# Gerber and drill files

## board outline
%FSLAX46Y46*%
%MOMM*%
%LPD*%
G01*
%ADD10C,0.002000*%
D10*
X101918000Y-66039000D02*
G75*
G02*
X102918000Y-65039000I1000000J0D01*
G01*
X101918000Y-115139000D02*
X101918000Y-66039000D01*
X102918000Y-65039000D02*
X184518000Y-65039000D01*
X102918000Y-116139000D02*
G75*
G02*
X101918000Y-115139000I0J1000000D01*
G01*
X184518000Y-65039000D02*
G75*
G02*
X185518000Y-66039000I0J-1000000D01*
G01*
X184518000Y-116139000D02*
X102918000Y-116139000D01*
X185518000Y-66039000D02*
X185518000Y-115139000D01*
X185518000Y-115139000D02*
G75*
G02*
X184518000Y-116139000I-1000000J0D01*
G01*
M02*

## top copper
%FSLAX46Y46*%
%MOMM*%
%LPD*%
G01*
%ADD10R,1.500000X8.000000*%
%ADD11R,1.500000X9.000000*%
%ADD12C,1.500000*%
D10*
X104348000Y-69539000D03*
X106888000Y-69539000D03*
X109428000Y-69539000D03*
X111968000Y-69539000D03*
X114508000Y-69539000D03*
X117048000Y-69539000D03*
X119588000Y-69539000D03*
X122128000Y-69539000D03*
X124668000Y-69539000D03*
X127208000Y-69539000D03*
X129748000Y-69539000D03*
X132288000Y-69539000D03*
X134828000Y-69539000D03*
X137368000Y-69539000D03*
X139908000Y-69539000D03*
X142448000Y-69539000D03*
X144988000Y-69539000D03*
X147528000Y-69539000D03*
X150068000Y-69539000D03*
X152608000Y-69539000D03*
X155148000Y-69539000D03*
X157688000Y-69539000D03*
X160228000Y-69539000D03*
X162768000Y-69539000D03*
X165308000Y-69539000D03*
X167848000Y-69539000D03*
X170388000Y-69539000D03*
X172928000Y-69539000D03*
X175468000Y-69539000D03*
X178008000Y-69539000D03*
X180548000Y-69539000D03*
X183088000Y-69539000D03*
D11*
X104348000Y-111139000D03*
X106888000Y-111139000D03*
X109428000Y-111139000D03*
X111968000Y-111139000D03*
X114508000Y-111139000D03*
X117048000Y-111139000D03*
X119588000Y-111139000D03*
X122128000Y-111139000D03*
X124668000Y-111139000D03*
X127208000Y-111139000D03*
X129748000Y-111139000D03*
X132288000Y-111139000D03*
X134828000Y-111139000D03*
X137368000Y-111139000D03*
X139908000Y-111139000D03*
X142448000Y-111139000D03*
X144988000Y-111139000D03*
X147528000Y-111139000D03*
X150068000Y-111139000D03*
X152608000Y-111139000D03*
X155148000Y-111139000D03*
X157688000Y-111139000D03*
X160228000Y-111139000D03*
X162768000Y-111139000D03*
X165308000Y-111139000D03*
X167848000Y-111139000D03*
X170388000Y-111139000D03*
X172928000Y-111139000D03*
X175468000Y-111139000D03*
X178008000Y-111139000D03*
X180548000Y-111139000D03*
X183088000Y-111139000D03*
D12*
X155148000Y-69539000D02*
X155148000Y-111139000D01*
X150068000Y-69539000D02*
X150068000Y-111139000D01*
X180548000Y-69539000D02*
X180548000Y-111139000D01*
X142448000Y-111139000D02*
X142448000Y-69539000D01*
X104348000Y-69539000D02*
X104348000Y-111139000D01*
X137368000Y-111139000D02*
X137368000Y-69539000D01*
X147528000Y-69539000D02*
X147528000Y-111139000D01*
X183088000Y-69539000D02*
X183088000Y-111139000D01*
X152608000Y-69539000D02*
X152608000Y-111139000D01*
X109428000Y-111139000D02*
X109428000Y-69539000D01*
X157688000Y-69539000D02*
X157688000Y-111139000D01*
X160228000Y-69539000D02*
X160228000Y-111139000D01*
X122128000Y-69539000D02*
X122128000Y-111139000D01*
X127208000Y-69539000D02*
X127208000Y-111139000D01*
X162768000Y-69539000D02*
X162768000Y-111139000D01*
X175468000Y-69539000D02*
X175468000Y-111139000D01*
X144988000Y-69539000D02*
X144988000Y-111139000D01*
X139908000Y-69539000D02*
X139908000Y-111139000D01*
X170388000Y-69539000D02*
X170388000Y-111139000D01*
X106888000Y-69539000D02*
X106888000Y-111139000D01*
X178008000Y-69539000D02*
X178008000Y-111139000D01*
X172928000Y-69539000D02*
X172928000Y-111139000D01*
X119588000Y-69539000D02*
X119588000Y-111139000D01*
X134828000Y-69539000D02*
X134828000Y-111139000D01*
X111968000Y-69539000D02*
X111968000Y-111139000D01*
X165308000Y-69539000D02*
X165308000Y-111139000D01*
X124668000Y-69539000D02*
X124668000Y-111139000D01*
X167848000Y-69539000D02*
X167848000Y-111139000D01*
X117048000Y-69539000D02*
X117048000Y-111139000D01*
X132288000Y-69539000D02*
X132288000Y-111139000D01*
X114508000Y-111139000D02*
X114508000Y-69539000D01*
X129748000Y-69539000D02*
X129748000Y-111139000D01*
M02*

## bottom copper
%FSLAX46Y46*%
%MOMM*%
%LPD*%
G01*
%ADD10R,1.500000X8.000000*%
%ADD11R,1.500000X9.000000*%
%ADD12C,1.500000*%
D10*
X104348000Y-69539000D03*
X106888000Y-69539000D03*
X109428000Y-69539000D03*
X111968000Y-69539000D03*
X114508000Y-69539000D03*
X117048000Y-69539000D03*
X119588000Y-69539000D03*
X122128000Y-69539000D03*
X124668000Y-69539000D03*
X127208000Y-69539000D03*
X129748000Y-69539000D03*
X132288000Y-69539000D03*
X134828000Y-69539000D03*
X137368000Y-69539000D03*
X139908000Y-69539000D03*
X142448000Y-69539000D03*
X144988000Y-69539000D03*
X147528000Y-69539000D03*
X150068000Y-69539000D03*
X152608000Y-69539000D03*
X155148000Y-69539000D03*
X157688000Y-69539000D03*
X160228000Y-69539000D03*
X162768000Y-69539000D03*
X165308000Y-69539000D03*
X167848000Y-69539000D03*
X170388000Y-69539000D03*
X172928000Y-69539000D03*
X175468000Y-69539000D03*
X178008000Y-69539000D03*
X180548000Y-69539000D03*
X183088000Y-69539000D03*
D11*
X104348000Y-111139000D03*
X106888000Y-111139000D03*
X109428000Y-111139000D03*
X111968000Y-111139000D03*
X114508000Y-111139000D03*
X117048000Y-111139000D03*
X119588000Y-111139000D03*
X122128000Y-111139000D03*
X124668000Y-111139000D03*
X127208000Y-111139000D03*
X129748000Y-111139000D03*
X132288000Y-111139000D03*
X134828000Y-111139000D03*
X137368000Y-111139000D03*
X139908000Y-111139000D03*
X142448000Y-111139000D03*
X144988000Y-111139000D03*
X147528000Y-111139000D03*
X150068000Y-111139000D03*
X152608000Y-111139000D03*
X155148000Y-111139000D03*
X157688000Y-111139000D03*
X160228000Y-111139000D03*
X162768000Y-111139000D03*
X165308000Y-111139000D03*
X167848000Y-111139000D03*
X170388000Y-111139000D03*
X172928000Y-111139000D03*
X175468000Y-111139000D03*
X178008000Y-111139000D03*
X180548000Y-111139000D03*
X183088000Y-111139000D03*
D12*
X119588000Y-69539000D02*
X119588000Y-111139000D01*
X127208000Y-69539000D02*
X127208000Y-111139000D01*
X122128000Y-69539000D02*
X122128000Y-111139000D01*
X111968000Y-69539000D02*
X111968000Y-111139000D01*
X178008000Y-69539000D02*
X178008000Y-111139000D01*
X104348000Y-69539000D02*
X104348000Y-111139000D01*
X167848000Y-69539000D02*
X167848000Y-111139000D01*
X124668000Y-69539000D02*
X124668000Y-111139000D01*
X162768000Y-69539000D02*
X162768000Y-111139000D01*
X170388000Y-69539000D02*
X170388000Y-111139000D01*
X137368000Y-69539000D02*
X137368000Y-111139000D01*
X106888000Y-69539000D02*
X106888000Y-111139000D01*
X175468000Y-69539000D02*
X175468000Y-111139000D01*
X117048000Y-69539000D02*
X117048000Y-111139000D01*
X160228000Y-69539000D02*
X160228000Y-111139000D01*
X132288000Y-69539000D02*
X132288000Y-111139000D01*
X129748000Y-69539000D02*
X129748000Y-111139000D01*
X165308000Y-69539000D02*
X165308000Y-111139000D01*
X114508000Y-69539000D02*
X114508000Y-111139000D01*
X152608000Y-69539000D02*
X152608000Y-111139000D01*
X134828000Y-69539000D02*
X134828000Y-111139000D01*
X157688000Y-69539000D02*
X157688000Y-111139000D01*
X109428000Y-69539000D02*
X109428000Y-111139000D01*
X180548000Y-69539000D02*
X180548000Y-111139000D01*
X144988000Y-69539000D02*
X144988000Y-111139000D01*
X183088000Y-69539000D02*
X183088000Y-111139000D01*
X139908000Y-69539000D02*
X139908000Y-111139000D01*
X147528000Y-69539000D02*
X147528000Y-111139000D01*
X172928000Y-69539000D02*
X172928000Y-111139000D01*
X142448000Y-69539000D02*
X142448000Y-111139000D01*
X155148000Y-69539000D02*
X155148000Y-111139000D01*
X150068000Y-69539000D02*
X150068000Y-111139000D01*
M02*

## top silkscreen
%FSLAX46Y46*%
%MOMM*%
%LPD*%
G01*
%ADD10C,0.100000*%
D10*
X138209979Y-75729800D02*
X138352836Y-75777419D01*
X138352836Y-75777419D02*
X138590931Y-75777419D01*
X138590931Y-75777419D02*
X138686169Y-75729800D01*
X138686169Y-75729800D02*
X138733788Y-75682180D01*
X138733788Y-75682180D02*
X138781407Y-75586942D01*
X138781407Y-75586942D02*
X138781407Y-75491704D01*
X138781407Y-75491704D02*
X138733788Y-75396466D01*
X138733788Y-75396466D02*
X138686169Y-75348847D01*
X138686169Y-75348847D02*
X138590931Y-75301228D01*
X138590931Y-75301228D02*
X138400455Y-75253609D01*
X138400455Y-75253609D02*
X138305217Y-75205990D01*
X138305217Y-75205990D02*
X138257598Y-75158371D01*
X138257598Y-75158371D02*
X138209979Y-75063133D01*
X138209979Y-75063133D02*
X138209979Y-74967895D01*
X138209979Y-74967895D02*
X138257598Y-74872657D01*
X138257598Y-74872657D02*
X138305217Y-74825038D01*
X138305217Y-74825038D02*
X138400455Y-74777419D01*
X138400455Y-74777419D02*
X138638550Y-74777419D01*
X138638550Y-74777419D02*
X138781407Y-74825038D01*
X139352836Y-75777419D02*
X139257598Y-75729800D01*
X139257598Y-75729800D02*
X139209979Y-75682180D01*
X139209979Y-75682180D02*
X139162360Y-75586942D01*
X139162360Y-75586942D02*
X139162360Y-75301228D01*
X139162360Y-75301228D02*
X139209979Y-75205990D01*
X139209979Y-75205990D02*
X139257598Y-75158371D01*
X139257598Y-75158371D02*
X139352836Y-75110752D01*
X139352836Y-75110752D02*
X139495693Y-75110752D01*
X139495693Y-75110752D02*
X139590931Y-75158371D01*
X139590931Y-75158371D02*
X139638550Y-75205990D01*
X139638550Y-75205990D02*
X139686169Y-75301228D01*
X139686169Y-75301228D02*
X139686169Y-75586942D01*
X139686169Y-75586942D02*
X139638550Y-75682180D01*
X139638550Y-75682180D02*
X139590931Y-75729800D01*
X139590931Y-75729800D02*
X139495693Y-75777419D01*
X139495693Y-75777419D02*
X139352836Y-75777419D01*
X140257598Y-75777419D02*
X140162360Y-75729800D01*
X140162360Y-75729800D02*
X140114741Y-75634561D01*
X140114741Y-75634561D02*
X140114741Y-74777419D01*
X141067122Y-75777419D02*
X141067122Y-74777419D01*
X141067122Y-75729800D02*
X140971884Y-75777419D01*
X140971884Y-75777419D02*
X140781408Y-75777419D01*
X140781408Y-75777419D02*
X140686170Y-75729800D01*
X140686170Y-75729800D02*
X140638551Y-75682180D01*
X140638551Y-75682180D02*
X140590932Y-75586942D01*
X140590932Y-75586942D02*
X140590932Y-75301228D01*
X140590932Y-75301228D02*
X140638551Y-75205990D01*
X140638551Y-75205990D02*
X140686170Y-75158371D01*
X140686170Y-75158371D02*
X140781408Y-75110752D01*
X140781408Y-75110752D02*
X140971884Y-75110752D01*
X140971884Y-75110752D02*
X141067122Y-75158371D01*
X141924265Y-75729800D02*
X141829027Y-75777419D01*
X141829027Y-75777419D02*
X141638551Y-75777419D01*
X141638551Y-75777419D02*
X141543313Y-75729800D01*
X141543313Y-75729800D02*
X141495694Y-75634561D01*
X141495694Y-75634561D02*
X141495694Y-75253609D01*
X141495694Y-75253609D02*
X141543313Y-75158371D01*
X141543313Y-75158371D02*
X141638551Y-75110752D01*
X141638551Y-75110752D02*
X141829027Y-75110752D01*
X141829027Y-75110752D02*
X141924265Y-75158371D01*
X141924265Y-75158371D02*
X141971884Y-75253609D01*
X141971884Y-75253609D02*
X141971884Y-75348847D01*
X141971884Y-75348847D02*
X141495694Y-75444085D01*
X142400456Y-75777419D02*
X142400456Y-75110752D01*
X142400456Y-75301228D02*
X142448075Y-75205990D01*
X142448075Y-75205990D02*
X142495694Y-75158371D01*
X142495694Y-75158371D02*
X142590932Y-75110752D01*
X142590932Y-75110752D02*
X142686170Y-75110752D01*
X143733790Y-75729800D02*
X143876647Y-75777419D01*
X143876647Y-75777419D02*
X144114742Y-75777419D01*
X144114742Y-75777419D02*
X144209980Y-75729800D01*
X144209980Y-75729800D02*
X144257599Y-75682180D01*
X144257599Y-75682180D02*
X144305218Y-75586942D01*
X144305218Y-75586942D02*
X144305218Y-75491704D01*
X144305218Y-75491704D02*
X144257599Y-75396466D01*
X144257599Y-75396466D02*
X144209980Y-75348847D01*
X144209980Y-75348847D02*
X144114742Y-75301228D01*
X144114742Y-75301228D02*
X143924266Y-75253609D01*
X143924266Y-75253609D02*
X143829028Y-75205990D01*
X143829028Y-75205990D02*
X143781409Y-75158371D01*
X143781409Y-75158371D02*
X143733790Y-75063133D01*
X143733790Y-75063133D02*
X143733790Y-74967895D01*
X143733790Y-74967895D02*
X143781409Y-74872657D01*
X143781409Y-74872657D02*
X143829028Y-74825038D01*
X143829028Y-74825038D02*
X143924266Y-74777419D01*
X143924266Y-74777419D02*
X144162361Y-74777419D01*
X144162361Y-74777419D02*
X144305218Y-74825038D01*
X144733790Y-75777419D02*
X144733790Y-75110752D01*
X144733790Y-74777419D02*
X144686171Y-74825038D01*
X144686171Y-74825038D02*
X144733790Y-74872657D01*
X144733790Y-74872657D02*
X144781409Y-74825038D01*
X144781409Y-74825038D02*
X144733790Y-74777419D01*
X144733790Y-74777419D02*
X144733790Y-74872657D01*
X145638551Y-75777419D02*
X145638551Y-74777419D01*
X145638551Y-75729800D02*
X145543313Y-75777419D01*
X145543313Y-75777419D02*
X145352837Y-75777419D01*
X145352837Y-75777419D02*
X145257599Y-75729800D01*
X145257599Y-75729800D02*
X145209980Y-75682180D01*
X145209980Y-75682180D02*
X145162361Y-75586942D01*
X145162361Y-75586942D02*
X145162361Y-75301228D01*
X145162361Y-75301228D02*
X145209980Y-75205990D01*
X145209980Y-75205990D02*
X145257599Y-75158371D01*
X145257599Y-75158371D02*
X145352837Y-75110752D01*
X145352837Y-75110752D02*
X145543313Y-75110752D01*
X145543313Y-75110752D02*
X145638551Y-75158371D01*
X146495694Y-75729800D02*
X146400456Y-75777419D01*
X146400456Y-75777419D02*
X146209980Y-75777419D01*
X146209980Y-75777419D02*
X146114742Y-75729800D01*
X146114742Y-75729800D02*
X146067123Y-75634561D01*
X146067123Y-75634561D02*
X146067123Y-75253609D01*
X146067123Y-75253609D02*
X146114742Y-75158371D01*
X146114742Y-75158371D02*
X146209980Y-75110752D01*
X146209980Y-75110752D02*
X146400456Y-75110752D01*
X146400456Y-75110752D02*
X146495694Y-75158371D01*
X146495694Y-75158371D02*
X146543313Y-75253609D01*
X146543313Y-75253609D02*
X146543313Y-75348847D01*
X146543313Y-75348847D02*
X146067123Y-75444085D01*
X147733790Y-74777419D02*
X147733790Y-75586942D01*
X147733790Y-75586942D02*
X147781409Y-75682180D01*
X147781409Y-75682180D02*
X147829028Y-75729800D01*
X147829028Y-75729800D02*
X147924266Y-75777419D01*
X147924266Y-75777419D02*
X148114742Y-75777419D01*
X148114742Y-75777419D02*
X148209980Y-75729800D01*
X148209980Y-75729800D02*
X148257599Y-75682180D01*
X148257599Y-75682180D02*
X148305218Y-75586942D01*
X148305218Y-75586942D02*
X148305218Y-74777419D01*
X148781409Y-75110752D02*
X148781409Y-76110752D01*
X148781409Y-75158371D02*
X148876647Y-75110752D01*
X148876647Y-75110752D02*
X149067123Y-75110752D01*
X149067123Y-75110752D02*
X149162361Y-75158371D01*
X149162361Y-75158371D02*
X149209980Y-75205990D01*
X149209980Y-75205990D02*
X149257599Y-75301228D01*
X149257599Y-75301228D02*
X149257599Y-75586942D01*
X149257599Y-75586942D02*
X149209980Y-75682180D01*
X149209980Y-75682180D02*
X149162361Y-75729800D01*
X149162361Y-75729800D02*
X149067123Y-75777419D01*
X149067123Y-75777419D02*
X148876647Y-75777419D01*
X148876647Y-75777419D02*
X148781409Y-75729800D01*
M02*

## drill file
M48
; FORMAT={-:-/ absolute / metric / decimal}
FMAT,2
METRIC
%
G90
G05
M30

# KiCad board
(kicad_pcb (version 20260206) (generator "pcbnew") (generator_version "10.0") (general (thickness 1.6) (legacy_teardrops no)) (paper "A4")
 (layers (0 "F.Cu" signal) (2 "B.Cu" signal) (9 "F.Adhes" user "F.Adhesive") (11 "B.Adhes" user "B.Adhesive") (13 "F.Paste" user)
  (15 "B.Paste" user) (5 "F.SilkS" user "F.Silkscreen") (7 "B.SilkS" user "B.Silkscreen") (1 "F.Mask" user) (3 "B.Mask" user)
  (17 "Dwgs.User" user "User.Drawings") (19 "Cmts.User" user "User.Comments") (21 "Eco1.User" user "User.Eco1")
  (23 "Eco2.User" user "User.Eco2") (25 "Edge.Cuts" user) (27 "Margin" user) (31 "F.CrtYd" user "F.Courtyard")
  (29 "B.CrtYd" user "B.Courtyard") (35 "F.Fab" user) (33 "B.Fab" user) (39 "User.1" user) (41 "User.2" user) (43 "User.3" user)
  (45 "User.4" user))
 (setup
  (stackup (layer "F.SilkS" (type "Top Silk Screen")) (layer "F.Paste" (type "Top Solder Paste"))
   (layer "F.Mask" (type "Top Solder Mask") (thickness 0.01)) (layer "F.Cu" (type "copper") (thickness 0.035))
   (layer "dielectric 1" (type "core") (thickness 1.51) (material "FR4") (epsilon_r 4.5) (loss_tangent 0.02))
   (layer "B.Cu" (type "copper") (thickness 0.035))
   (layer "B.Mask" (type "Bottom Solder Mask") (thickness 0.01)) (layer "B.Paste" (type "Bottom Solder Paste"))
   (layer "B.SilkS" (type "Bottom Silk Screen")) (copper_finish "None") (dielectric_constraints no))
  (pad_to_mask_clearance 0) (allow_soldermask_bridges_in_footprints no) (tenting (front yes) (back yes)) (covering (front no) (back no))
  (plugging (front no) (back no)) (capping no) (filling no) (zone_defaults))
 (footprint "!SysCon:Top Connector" (layer "F.Cu") (at 143.718 69.539)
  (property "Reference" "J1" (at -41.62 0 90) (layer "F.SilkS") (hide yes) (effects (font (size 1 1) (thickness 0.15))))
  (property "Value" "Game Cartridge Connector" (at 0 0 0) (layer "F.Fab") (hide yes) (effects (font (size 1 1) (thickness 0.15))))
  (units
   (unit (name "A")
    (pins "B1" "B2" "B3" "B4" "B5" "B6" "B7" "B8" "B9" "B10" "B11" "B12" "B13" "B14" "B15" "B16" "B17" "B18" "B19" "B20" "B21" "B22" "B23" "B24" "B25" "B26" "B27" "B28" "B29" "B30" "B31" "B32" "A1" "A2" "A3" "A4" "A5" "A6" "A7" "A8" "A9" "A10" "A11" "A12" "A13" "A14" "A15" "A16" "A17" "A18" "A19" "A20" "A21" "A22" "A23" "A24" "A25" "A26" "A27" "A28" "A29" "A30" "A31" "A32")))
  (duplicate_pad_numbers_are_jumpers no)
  (pad "A1" smd rect (at -39.37 0) (size 1.5 8) (layers "B.Cu" "B.Mask") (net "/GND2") (thermal_bridge_angle 45))
  (pad "A2" smd rect (at -36.83 0) (size 1.5 8) (layers "B.Cu" "B.Mask") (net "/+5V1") (thermal_bridge_angle 45))
  (pad "A3" smd rect (at -34.29 0) (size 1.5 8) (layers "B.Cu" "B.Mask") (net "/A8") (thermal_bridge_angle 45))
  (pad "A4" smd rect (at -31.75 0) (size 1.5 8) (layers "B.Cu" "B.Mask") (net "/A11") (thermal_bridge_angle 45))
  (pad "A5" smd rect (at -29.21 0) (size 1.5 8) (layers "B.Cu" "B.Mask") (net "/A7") (thermal_bridge_angle 45))
  (pad "A6" smd rect (at -26.67 0) (size 1.5 8) (layers "B.Cu" "B.Mask") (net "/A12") (thermal_bridge_angle 45))
  (pad "A7" smd rect (at -24.13 0) (size 1.5 8) (layers "B.Cu" "B.Mask") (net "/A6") (thermal_bridge_angle 45))
  (pad "A8" smd rect (at -21.59 0) (size 1.5 8) (layers "B.Cu" "B.Mask") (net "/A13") (thermal_bridge_angle 45))
  (pad "A9" smd rect (at -19.05 0) (size 1.5 8) (layers "B.Cu" "B.Mask") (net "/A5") (thermal_bridge_angle 45))
  (pad "A10" smd rect (at -16.51 0) (size 1.5 8) (layers "B.Cu" "B.Mask") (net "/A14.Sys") (thermal_bridge_angle 45))
  (pad "A11" smd rect (at -13.97 0) (size 1.5 8) (layers "B.Cu" "B.Mask") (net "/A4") (thermal_bridge_angle 45))
  (pad "A12" smd rect (at -11.43 0) (size 1.5 8) (layers "B.Cu" "B.Mask") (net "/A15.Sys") (thermal_bridge_angle 45))
  (pad "A13" smd rect (at -8.89 0) (size 1.5 8) (layers "B.Cu" "B.Mask") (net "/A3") (thermal_bridge_angle 45))
  (pad "A14" smd rect (at -6.35 0) (size 1.5 8) (layers "B.Cu" "B.Mask") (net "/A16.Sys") (thermal_bridge_angle 45))
  (pad "A15" smd rect (at -3.81 0) (size 1.5 8) (layers "B.Cu" "B.Mask") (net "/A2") (thermal_bridge_angle 45))
  (pad "A16" smd rect (at -1.27 0) (size 1.5 8) (layers "B.Cu" "B.Mask") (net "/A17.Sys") (thermal_bridge_angle 45))
  (pad "A17" smd rect (at 1.27 0) (size 1.5 8) (layers "B.Cu" "B.Mask") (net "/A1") (thermal_bridge_angle 45))
  (pad "A18" smd rect (at 3.81 0) (size 1.5 8) (layers "B.Cu" "B.Mask") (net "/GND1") (thermal_bridge_angle 45))
  (pad "A19" smd rect (at 6.35 0) (size 1.5 8) (layers "B.Cu" "B.Mask") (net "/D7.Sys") (thermal_bridge_angle 45))
  (pad "A20" smd rect (at 8.89 0) (size 1.5 8) (layers "B.Cu" "B.Mask") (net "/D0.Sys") (thermal_bridge_angle 45))
  (pad "A21" smd rect (at 11.43 0) (size 1.5 8) (layers "B.Cu" "B.Mask") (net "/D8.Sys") (thermal_bridge_angle 45))
  (pad "A22" smd rect (at 13.97 0) (size 1.5 8) (layers "B.Cu" "B.Mask") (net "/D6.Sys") (thermal_bridge_angle 45))
  (pad "A23" smd rect (at 16.51 0) (size 1.5 8) (layers "B.Cu" "B.Mask") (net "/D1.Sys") (thermal_bridge_angle 45))
  (pad "A24" smd rect (at 19.05 0) (size 1.5 8) (layers "B.Cu" "B.Mask") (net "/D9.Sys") (thermal_bridge_angle 45))
  (pad "A25" smd rect (at 21.59 0) (size 1.5 8) (layers "B.Cu" "B.Mask") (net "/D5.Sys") (thermal_bridge_angle 45))
  (pad "A26" smd rect (at 24.13 0) (size 1.5 8) (layers "B.Cu" "B.Mask") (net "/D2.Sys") (thermal_bridge_angle 45))
  (pad "A27" smd rect (at 26.67 0) (size 1.5 8) (layers "B.Cu" "B.Mask") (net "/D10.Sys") (thermal_bridge_angle 45))
  (pad "A28" smd rect (at 29.21 0) (size 1.5 8) (layers "B.Cu" "B.Mask") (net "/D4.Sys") (thermal_bridge_angle 45))
  (pad "A29" smd rect (at 31.75 0) (size 1.5 8) (layers "B.Cu" "B.Mask") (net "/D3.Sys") (thermal_bridge_angle 45))
  (pad "A30" smd rect (at 34.29 0) (size 1.5 8) (layers "B.Cu" "B.Mask") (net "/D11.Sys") (thermal_bridge_angle 45))
  (pad "A31" smd rect (at 36.83 0) (size 1.5 8) (layers "B.Cu" "B.Mask") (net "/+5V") (thermal_bridge_angle 45))
  (pad "A32" smd rect (at 39.37 0) (size 1.5 8) (layers "B.Cu" "B.Mask") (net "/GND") (thermal_bridge_angle 45))
  (pad "B1" smd rect (at -39.37 0) (size 1.5 8) (layers "F.Cu" "F.Mask") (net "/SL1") (thermal_bridge_angle 45))
  (pad "B2" smd rect (at -36.83 0) (size 1.5 8) (layers "F.Cu" "F.Mask") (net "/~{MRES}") (thermal_bridge_angle 45))
  (pad "B3" smd rect (at -34.29 0) (size 1.5 8) (layers "F.Cu" "F.Mask") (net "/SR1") (thermal_bridge_angle 45))
  (pad "B4" smd rect (at -31.75 0) (size 1.5 8) (layers "F.Cu" "F.Mask") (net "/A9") (thermal_bridge_angle 45))
  (pad "B5" smd rect (at -29.21 0) (size 1.5 8) (layers "F.Cu" "F.Mask") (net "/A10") (thermal_bridge_angle 45))
  (pad "B6" smd rect (at -26.67 0) (size 1.5 8) (layers "F.Cu" "F.Mask") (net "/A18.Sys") (thermal_bridge_angle 45))
  (pad "B7" smd rect (at -24.13 0) (size 1.5 8) (layers "F.Cu" "F.Mask") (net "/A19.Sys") (thermal_bridge_angle 45))
  (pad "B8" smd rect (at -21.59 0) (size 1.5 8) (layers "F.Cu" "F.Mask") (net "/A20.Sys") (thermal_bridge_angle 45))
  (pad "B9" smd rect (at -19.05 0) (size 1.5 8) (layers "F.Cu" "F.Mask") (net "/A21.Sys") (thermal_bridge_angle 45))
  (pad "B10" smd rect (at -16.51 0) (size 1.5 8) (layers "F.Cu" "F.Mask") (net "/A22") (thermal_bridge_angle 45))
  (pad "B11" smd rect (at -13.97 0) (size 1.5 8) (layers "F.Cu" "F.Mask") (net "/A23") (thermal_bridge_angle 45))
  (pad "B12" smd rect (at -11.43 0) (size 1.5 8) (layers "F.Cu" "F.Mask") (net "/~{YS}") (thermal_bridge_angle 45))
  (pad "B13" smd rect (at -8.89 0) (size 1.5 8) (layers "F.Cu" "F.Mask") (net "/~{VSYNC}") (thermal_bridge_angle 45))
  (pad "B14" smd rect (at -6.35 0) (size 1.5 8) (layers "F.Cu" "F.Mask") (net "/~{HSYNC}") (thermal_bridge_angle 45))
  (pad "B15" smd rect (at -3.81 0) (size 1.5 8) (layers "F.Cu" "F.Mask") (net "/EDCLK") (thermal_bridge_angle 45))
  (pad "B16" smd rect (at -1.27 0) (size 1.5 8) (layers "F.Cu" "F.Mask") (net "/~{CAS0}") (thermal_bridge_angle 45))
  (pad "B17" smd rect (at 1.27 0) (size 1.5 8) (layers "F.Cu" "F.Mask") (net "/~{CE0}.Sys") (thermal_bridge_angle 45))
  (pad "B18" smd rect (at 3.81 0) (size 1.5 8) (layers "F.Cu" "F.Mask") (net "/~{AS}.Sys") (thermal_bridge_angle 45))
  (pad "B19" smd rect (at 6.35 0) (size 1.5 8) (layers "F.Cu" "F.Mask") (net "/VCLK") (thermal_bridge_angle 45))
  (pad "B20" smd rect (at 8.89 0) (size 1.5 8) (layers "F.Cu" "F.Mask") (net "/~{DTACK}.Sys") (thermal_bridge_angle 45))
  (pad "B21" smd rect (at 11.43 0) (size 1.5 8) (layers "F.Cu" "F.Mask") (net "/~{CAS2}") (thermal_bridge_angle 45))
  (pad "B22" smd rect (at 13.97 0) (size 1.5 8) (layers "F.Cu" "F.Mask") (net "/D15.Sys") (thermal_bridge_angle 45))
  (pad "B23" smd rect (at 16.51 0) (size 1.5 8) (layers "F.Cu" "F.Mask") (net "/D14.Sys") (thermal_bridge_angle 45))
  (pad "B24" smd rect (at 19.05 0) (size 1.5 8) (layers "F.Cu" "F.Mask") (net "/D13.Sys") (thermal_bridge_angle 45))
  (pad "B25" smd rect (at 21.59 0) (size 1.5 8) (layers "F.Cu" "F.Mask") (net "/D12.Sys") (thermal_bridge_angle 45))
  (pad "B26" smd rect (at 24.13 0) (size 1.5 8) (layers "F.Cu" "F.Mask") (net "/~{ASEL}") (thermal_bridge_angle 45))
  (pad "B27" smd rect (at 26.67 0) (size 1.5 8) (layers "F.Cu" "F.Mask") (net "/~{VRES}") (thermal_bridge_angle 45))
  (pad "B28" smd rect (at 29.21 0) (size 1.5 8) (layers "F.Cu" "F.Mask") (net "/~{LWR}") (thermal_bridge_angle 45))
  (pad "B29" smd rect (at 31.75 0) (size 1.5 8) (layers "F.Cu" "F.Mask") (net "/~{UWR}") (thermal_bridge_angle 45))
  (pad "B30" smd rect (at 34.29 0) (size 1.5 8) (layers "F.Cu" "F.Mask") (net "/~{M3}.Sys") (thermal_bridge_angle 45))
  (pad "B31" smd rect (at 36.83 0) (size 1.5 8) (layers "F.Cu" "F.Mask") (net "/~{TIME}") (thermal_bridge_angle 45))
  (pad "B32" smd rect (at 39.37 0) (size 1.5 8) (layers "F.Cu" "F.Mask") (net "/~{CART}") (thermal_bridge_angle 45)))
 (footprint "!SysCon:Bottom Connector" (layer "F.Cu") (at 143.718 111.139)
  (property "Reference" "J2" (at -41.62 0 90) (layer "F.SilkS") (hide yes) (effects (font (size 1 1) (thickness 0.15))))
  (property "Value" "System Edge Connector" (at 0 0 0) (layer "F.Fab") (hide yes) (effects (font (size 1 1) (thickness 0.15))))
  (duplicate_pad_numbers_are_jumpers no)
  (pad "A1" smd rect (at -39.37 0) (size 1.5 9) (layers "B.Cu" "B.Mask") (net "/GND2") (thermal_bridge_angle 45))
  (pad "A2" smd rect (at -36.83 0) (size 1.5 9) (layers "B.Cu" "B.Mask") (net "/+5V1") (thermal_bridge_angle 45))
  (pad "A3" smd rect (at -34.29 0) (size 1.5 9) (layers "B.Cu" "B.Mask") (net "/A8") (thermal_bridge_angle 45))
  (pad "A4" smd rect (at -31.75 0) (size 1.5 9) (layers "B.Cu" "B.Mask") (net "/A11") (thermal_bridge_angle 45))
  (pad "A5" smd rect (at -29.21 0) (size 1.5 9) (layers "B.Cu" "B.Mask") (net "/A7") (thermal_bridge_angle 45))
  (pad "A6" smd rect (at -26.67 0) (size 1.5 9) (layers "B.Cu" "B.Mask") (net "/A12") (thermal_bridge_angle 45))
  (pad "A7" smd rect (at -24.13 0) (size 1.5 9) (layers "B.Cu" "B.Mask") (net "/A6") (thermal_bridge_angle 45))
  (pad "A8" smd rect (at -21.59 0) (size 1.5 9) (layers "B.Cu" "B.Mask") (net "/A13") (thermal_bridge_angle 45))
  (pad "A9" smd rect (at -19.05 0) (size 1.5 9) (layers "B.Cu" "B.Mask") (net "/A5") (thermal_bridge_angle 45))
  (pad "A10" smd rect (at -16.51 0) (size 1.5 9) (layers "B.Cu" "B.Mask") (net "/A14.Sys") (thermal_bridge_angle 45))
  (pad "A11" smd rect (at -13.97 0) (size 1.5 9) (layers "B.Cu" "B.Mask") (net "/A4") (thermal_bridge_angle 45))
  (pad "A12" smd rect (at -11.43 0) (size 1.5 9) (layers "B.Cu" "B.Mask") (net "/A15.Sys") (thermal_bridge_angle 45))
  (pad "A13" smd rect (at -8.89 0) (size 1.5 9) (layers "B.Cu" "B.Mask") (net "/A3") (thermal_bridge_angle 45))
  (pad "A14" smd rect (at -6.35 0) (size 1.5 9) (layers "B.Cu" "B.Mask") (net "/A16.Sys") (thermal_bridge_angle 45))
  (pad "A15" smd rect (at -3.81 0) (size 1.5 9) (layers "B.Cu" "B.Mask") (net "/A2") (thermal_bridge_angle 45))
  (pad "A16" smd rect (at -1.27 0) (size 1.5 9) (layers "B.Cu" "B.Mask") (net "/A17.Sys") (thermal_bridge_angle 45))
  (pad "A17" smd rect (at 1.27 0) (size 1.5 9) (layers "B.Cu" "B.Mask") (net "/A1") (thermal_bridge_angle 45))
  (pad "A18" smd rect (at 3.81 0) (size 1.5 9) (layers "B.Cu" "B.Mask") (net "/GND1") (thermal_bridge_angle 45))
  (pad "A19" smd rect (at 6.35 0) (size 1.5 9) (layers "B.Cu" "B.Mask") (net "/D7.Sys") (thermal_bridge_angle 45))
  (pad "A20" smd rect (at 8.89 0) (size 1.5 9) (layers "B.Cu" "B.Mask") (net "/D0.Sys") (thermal_bridge_angle 45))
  (pad "A21" smd rect (at 11.43 0) (size 1.5 9) (layers "B.Cu" "B.Mask") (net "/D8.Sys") (thermal_bridge_angle 45))
  (pad "A22" smd rect (at 13.97 0) (size 1.5 9) (layers "B.Cu" "B.Mask") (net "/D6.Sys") (thermal_bridge_angle 45))
  (pad "A23" smd rect (at 16.51 0) (size 1.5 9) (layers "B.Cu" "B.Mask") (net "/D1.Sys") (thermal_bridge_angle 45))
  (pad "A24" smd rect (at 19.05 0) (size 1.5 9) (layers "B.Cu" "B.Mask") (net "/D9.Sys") (thermal_bridge_angle 45))
  (pad "A25" smd rect (at 21.59 0) (size 1.5 9) (layers "B.Cu" "B.Mask") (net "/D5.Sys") (thermal_bridge_angle 45))
  (pad "A26" smd rect (at 24.13 0) (size 1.5 9) (layers "B.Cu" "B.Mask") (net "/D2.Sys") (thermal_bridge_angle 45))
  (pad "A27" smd rect (at 26.67 0) (size 1.5 9) (layers "B.Cu" "B.Mask") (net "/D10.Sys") (thermal_bridge_angle 45))
  (pad "A28" smd rect (at 29.21 0) (size 1.5 9) (layers "B.Cu" "B.Mask") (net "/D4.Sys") (thermal_bridge_angle 45))
  (pad "A29" smd rect (at 31.75 0) (size 1.5 9) (layers "B.Cu" "B.Mask") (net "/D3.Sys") (thermal_bridge_angle 45))
  (pad "A30" smd rect (at 34.29 0) (size 1.5 9) (layers "B.Cu" "B.Mask") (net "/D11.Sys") (thermal_bridge_angle 45))
  (pad "A31" smd rect (at 36.83 0) (size 1.5 9) (layers "B.Cu" "B.Mask") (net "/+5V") (thermal_bridge_angle 45))
  (pad "A32" smd rect (at 39.37 0) (size 1.5 9) (layers "B.Cu" "B.Mask") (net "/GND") (thermal_bridge_angle 45))
  (pad "B1" smd rect (at -39.37 0) (size 1.5 9) (layers "F.Cu" "F.Mask") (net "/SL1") (thermal_bridge_angle 45))
  (pad "B2" smd rect (at -36.83 0) (size 1.5 9) (layers "F.Cu" "F.Mask") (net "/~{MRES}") (thermal_bridge_angle 45))
  (pad "B3" smd rect (at -34.29 0) (size 1.5 9) (layers "F.Cu" "F.Mask") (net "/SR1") (thermal_bridge_angle 45))
  (pad "B4" smd rect (at -31.75 0) (size 1.5 9) (layers "F.Cu" "F.Mask") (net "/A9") (thermal_bridge_angle 45))
  (pad "B5" smd rect (at -29.21 0) (size 1.5 9) (layers "F.Cu" "F.Mask") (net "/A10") (thermal_bridge_angle 45))
  (pad "B6" smd rect (at -26.67 0) (size 1.5 9) (layers "F.Cu" "F.Mask") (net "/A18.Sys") (thermal_bridge_angle 45))
  (pad "B7" smd rect (at -24.13 0) (size 1.5 9) (layers "F.Cu" "F.Mask") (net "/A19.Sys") (thermal_bridge_angle 45))
  (pad "B8" smd rect (at -21.59 0) (size 1.5 9) (layers "F.Cu" "F.Mask") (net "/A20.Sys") (thermal_bridge_angle 45))
  (pad "B9" smd rect (at -19.05 0) (size 1.5 9) (layers "F.Cu" "F.Mask") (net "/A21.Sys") (thermal_bridge_angle 45))
  (pad "B10" smd rect (at -16.51 0) (size 1.5 9) (layers "F.Cu" "F.Mask") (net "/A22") (thermal_bridge_angle 45))
  (pad "B11" smd rect (at -13.97 0) (size 1.5 9) (layers "F.Cu" "F.Mask") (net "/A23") (thermal_bridge_angle 45))
  (pad "B12" smd rect (at -11.43 0) (size 1.5 9) (layers "F.Cu" "F.Mask") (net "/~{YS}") (thermal_bridge_angle 45))
  (pad "B13" smd rect (at -8.89 0) (size 1.5 9) (layers "F.Cu" "F.Mask") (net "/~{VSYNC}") (thermal_bridge_angle 45))
  (pad "B14" smd rect (at -6.35 0) (size 1.5 9) (layers "F.Cu" "F.Mask") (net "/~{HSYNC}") (thermal_bridge_angle 45))
  (pad "B15" smd rect (at -3.81 0) (size 1.5 9) (layers "F.Cu" "F.Mask") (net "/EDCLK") (thermal_bridge_angle 45))
  (pad "B16" smd rect (at -1.27 0) (size 1.5 9) (layers "F.Cu" "F.Mask") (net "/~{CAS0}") (thermal_bridge_angle 45))
  (pad "B17" smd rect (at 1.27 0) (size 1.5 9) (layers "F.Cu" "F.Mask") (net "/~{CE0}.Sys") (thermal_bridge_angle 45))
  (pad "B18" smd rect (at 3.81 0) (size 1.5 9) (layers "F.Cu" "F.Mask") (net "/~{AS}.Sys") (thermal_bridge_angle 45))
  (pad "B19" smd rect (at 6.35 0) (size 1.5 9) (layers "F.Cu" "F.Mask") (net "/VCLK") (thermal_bridge_angle 45))
  (pad "B20" smd rect (at 8.89 0) (size 1.5 9) (layers "F.Cu" "F.Mask") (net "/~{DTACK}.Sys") (thermal_bridge_angle 45))
  (pad "B21" smd rect (at 11.43 0) (size 1.5 9) (layers "F.Cu" "F.Mask") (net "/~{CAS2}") (thermal_bridge_angle 45))
  (pad "B22" smd rect (at 13.97 0) (size 1.5 9) (layers "F.Cu" "F.Mask") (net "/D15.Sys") (thermal_bridge_angle 45))
  (pad "B23" smd rect (at 16.51 0) (size 1.5 9) (layers "F.Cu" "F.Mask") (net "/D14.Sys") (thermal_bridge_angle 45))
  (pad "B24" smd rect (at 19.05 0) (size 1.5 9) (layers "F.Cu" "F.Mask") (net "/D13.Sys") (thermal_bridge_angle 45))
  (pad "B25" smd rect (at 21.59 0) (size 1.5 9) (layers "F.Cu" "F.Mask") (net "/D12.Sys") (thermal_bridge_angle 45))
  (pad "B26" smd rect (at 24.13 0) (size 1.5 9) (layers "F.Cu" "F.Mask") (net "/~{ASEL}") (thermal_bridge_angle 45))
  (pad "B27" smd rect (at 26.67 0) (size 1.5 9) (layers "F.Cu" "F.Mask") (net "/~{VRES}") (thermal_bridge_angle 45))
  (pad "B28" smd rect (at 29.21 0) (size 1.5 9) (layers "F.Cu" "F.Mask") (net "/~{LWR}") (thermal_bridge_angle 45))
  (pad "B29" smd rect (at 31.75 0) (size 1.5 9) (layers "F.Cu" "F.Mask") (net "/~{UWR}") (thermal_bridge_angle 45))
  (pad "B30" smd rect (at 34.29 0) (size 1.5 9) (layers "F.Cu" "F.Mask") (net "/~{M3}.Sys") (thermal_bridge_angle 45))
  (pad "B31" smd rect (at 36.83 0) (size 1.5 9) (layers "F.Cu" "F.Mask") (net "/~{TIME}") (thermal_bridge_angle 45))
  (pad "B32" smd rect (at 39.37 0) (size 1.5 9) (layers "F.Cu" "F.Mask") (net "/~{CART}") (thermal_bridge_angle 45)))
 (gr_arc (start 101.918 66.039) (mid 102.210893 65.331893) (end 102.918 65.039) (stroke (width 0.002) (type default)) (layer "Edge.Cuts"))
 (gr_line (start 101.918 115.139) (end 101.918 66.039) (stroke (width 0.002) (type default)) (layer "Edge.Cuts"))
 (gr_line (start 102.918 65.039) (end 184.518 65.039) (stroke (width 0.002) (type default)) (layer "Edge.Cuts"))
 (gr_arc (start 102.918 116.139) (mid 102.210893 115.846107) (end 101.918 115.139) (stroke (width 0.002) (type default)) (layer "Edge.Cuts"))
 (gr_arc (start 184.518 65.039) (mid 185.225107 65.331893) (end 185.518 66.039) (stroke (width 0.002) (type default)) (layer "Edge.Cuts"))
 (gr_line (start 184.518 116.139) (end 102.918 116.139) (stroke (width 0.002) (type default)) (layer "Edge.Cuts"))
 (gr_line (start 185.518 66.039) (end 185.518 115.139) (stroke (width 0.002) (type default)) (layer "Edge.Cuts"))
 (gr_arc (start 185.518 115.139) (mid 185.225107 115.846107) (end 184.518 116.139) (stroke (width 0.002) (type default)) (layer "Edge.Cuts"))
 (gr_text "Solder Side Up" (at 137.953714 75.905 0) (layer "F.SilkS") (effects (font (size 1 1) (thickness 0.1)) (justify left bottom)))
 (segment (start 155.148 69.539) (end 155.148 111.139) (width 1.5) (layer "F.Cu") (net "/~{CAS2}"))
 (segment (start 119.588 69.539) (end 119.588 111.139) (width 1.5) (layer "B.Cu") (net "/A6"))
 (segment (start 127.208 69.539) (end 127.208 111.139) (width 1.5) (layer "B.Cu") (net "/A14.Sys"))
 (segment (start 150.068 69.539) (end 150.068 111.139) (width 1.5) (layer "F.Cu") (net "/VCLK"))
 (segment (start 180.548 69.539) (end 180.548 111.139) (width 1.5) (layer "F.Cu") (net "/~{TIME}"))
 (segment (start 122.128 69.539) (end 122.128 111.139) (width 1.5) (layer "B.Cu") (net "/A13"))
 (segment (start 142.448 111.139) (end 142.448 69.539) (width 1.5) (layer "F.Cu") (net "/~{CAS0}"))
 (segment (start 111.968 69.539) (end 111.968 111.139) (width 1.5) (layer "B.Cu") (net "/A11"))
 (segment (start 104.348 69.539) (end 104.348 111.139) (width 1.5) (layer "F.Cu") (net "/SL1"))
 (segment (start 137.368 111.139) (end 137.368 69.539) (width 1.5) (layer "F.Cu") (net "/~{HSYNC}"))
 (segment (start 178.008 69.539) (end 178.008 111.139) (width 1.5) (layer "B.Cu") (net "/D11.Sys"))
 (segment (start 147.528 69.539) (end 147.528 111.139) (width 1.5) (layer "F.Cu") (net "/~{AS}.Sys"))
 (segment (start 104.348 69.539) (end 104.348 111.139) (width 1.5) (layer "B.Cu") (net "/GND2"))
 (segment (start 183.088 69.539) (end 183.088 111.139) (width 1.5) (layer "F.Cu") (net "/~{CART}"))
 (segment (start 167.848 69.539) (end 167.848 111.139) (width 1.5) (layer "B.Cu") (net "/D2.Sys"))
 (segment (start 152.608 69.539) (end 152.608 111.139) (width 1.5) (layer "F.Cu") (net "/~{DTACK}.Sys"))
 (segment (start 124.668 69.539) (end 124.668 111.139) (width 1.5) (layer "B.Cu") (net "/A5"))
 (segment (start 109.428 111.139) (end 109.428 69.539) (width 1.5) (layer "F.Cu") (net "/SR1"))
 (segment (start 157.688 69.539) (end 157.688 111.139) (width 1.5) (layer "F.Cu") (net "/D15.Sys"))
 (segment (start 162.768 69.539) (end 162.768 111.139) (width 1.5) (layer "B.Cu") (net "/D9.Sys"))
 (segment (start 170.388 69.539) (end 170.388 111.139) (width 1.5) (layer "B.Cu") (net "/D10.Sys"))
 (segment (start 160.228 69.539) (end 160.228 111.139) (width 1.5) (layer "F.Cu") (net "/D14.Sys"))
 (segment (start 122.128 69.539) (end 122.128 111.139) (width 1.5) (layer "F.Cu") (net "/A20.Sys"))
 (segment (start 127.208 69.539) (end 127.208 111.139) (width 1.5) (layer "F.Cu") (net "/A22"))
 (segment (start 162.768 69.539) (end 162.768 111.139) (width 1.5) (layer "F.Cu") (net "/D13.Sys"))
 (segment (start 137.368 69.539) (end 137.368 111.139) (width 1.5) (layer "B.Cu") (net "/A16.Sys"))
 (segment (start 106.888 69.539) (end 106.888 111.139) (width 1.5) (layer "B.Cu") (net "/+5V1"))
 (segment (start 175.468 69.539) (end 175.468 111.139) (width 1.5) (layer "B.Cu") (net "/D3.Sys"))
 (segment (start 117.048 69.539) (end 117.048 111.139) (width 1.5) (layer "B.Cu") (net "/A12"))
 (segment (start 175.468 69.539) (end 175.468 111.139) (width 1.5) (layer "F.Cu") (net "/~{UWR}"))
 (segment (start 144.988 69.539) (end 144.988 111.139) (width 1.5) (layer "F.Cu") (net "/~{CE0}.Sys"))
 (segment (start 160.228 69.539) (end 160.228 111.139) (width 1.5) (layer "B.Cu") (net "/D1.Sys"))
 (segment (start 139.908 69.539) (end 139.908 111.139) (width 1.5) (layer "F.Cu") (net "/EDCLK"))
 (segment (start 132.288 69.539) (end 132.288 111.139) (width 1.5) (layer "B.Cu") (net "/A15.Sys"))
 (segment (start 170.388 69.539) (end 170.388 111.139) (width 1.5) (layer "F.Cu") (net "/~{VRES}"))
 (segment (start 106.888 69.539) (end 106.888 111.139) (width 1.5) (layer "F.Cu") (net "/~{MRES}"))
 (segment (start 178.008 69.539) (end 178.008 111.139) (width 1.5) (layer "F.Cu") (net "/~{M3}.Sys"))
 (segment (start 172.928 69.539) (end 172.928 111.139) (width 1.5) (layer "F.Cu") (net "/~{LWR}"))
 (segment (start 129.748 69.539) (end 129.748 111.139) (width 1.5) (layer "B.Cu") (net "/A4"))
 (segment (start 165.308 69.539) (end 165.308 111.139) (width 1.5) (layer "B.Cu") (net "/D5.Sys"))
 (segment (start 119.588 69.539) (end 119.588 111.139) (width 1.5) (layer "F.Cu") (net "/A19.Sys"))
 (segment (start 114.508 69.539) (end 114.508 111.139) (width 1.5) (layer "B.Cu") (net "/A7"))
 (segment (start 152.608 69.539) (end 152.608 111.139) (width 1.5) (layer "B.Cu") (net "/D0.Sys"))
 (segment (start 134.828 69.539) (end 134.828 111.139) (width 1.5) (layer "B.Cu") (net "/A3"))
 (segment (start 157.688 69.539) (end 157.688 111.139) (width 1.5) (layer "B.Cu") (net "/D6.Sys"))
 (segment (start 109.428 69.539) (end 109.428 111.139) (width 1.5) (layer "B.Cu") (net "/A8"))
 (segment (start 134.828 69.539) (end 134.828 111.139) (width 1.5) (layer "F.Cu") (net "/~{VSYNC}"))
 (segment (start 180.548 69.539) (end 180.548 111.139) (width 1.5) (layer "B.Cu") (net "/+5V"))
 (segment (start 111.968 69.539) (end 111.968 111.139) (width 1.5) (layer "F.Cu") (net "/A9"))
 (segment (start 144.988 69.539) (end 144.988 111.139) (width 1.5) (layer "B.Cu") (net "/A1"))
 (segment (start 183.088 69.539) (end 183.088 111.139) (width 1.5) (layer "B.Cu") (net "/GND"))
 (segment (start 139.908 69.539) (end 139.908 111.139) (width 1.5) (layer "B.Cu") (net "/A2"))
 (segment (start 165.308 69.539) (end 165.308 111.139) (width 1.5) (layer "F.Cu") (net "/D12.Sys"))
 (segment (start 147.528 69.539) (end 147.528 111.139) (width 1.5) (layer "B.Cu") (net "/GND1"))
 (segment (start 124.668 69.539) (end 124.668 111.139) (width 1.5) (layer "F.Cu") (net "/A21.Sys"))
 (segment (start 167.848 69.539) (end 167.848 111.139) (width 1.5) (layer "F.Cu") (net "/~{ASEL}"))
 (segment (start 117.048 69.539) (end 117.048 111.139) (width 1.5) (layer "F.Cu") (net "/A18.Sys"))
 (segment (start 172.928 69.539) (end 172.928 111.139) (width 1.5) (layer "B.Cu") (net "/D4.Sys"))
 (segment (start 142.448 69.539) (end 142.448 111.139) (width 1.5) (layer "B.Cu") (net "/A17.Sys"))
 (segment (start 155.148 69.539) (end 155.148 111.139) (width 1.5) (layer "B.Cu") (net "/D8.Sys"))
 (segment (start 132.288 69.539) (end 132.288 111.139) (width 1.5) (layer "F.Cu") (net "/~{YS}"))
 (segment (start 114.508 111.139) (end 114.508 69.539) (width 1.5) (layer "F.Cu") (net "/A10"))
 (segment (start 129.748 69.539) (end 129.748 111.139) (width 1.5) (layer "F.Cu") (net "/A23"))
 (segment (start 150.068 69.539) (end 150.068 111.139) (width 1.5) (layer "B.Cu") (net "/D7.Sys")))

